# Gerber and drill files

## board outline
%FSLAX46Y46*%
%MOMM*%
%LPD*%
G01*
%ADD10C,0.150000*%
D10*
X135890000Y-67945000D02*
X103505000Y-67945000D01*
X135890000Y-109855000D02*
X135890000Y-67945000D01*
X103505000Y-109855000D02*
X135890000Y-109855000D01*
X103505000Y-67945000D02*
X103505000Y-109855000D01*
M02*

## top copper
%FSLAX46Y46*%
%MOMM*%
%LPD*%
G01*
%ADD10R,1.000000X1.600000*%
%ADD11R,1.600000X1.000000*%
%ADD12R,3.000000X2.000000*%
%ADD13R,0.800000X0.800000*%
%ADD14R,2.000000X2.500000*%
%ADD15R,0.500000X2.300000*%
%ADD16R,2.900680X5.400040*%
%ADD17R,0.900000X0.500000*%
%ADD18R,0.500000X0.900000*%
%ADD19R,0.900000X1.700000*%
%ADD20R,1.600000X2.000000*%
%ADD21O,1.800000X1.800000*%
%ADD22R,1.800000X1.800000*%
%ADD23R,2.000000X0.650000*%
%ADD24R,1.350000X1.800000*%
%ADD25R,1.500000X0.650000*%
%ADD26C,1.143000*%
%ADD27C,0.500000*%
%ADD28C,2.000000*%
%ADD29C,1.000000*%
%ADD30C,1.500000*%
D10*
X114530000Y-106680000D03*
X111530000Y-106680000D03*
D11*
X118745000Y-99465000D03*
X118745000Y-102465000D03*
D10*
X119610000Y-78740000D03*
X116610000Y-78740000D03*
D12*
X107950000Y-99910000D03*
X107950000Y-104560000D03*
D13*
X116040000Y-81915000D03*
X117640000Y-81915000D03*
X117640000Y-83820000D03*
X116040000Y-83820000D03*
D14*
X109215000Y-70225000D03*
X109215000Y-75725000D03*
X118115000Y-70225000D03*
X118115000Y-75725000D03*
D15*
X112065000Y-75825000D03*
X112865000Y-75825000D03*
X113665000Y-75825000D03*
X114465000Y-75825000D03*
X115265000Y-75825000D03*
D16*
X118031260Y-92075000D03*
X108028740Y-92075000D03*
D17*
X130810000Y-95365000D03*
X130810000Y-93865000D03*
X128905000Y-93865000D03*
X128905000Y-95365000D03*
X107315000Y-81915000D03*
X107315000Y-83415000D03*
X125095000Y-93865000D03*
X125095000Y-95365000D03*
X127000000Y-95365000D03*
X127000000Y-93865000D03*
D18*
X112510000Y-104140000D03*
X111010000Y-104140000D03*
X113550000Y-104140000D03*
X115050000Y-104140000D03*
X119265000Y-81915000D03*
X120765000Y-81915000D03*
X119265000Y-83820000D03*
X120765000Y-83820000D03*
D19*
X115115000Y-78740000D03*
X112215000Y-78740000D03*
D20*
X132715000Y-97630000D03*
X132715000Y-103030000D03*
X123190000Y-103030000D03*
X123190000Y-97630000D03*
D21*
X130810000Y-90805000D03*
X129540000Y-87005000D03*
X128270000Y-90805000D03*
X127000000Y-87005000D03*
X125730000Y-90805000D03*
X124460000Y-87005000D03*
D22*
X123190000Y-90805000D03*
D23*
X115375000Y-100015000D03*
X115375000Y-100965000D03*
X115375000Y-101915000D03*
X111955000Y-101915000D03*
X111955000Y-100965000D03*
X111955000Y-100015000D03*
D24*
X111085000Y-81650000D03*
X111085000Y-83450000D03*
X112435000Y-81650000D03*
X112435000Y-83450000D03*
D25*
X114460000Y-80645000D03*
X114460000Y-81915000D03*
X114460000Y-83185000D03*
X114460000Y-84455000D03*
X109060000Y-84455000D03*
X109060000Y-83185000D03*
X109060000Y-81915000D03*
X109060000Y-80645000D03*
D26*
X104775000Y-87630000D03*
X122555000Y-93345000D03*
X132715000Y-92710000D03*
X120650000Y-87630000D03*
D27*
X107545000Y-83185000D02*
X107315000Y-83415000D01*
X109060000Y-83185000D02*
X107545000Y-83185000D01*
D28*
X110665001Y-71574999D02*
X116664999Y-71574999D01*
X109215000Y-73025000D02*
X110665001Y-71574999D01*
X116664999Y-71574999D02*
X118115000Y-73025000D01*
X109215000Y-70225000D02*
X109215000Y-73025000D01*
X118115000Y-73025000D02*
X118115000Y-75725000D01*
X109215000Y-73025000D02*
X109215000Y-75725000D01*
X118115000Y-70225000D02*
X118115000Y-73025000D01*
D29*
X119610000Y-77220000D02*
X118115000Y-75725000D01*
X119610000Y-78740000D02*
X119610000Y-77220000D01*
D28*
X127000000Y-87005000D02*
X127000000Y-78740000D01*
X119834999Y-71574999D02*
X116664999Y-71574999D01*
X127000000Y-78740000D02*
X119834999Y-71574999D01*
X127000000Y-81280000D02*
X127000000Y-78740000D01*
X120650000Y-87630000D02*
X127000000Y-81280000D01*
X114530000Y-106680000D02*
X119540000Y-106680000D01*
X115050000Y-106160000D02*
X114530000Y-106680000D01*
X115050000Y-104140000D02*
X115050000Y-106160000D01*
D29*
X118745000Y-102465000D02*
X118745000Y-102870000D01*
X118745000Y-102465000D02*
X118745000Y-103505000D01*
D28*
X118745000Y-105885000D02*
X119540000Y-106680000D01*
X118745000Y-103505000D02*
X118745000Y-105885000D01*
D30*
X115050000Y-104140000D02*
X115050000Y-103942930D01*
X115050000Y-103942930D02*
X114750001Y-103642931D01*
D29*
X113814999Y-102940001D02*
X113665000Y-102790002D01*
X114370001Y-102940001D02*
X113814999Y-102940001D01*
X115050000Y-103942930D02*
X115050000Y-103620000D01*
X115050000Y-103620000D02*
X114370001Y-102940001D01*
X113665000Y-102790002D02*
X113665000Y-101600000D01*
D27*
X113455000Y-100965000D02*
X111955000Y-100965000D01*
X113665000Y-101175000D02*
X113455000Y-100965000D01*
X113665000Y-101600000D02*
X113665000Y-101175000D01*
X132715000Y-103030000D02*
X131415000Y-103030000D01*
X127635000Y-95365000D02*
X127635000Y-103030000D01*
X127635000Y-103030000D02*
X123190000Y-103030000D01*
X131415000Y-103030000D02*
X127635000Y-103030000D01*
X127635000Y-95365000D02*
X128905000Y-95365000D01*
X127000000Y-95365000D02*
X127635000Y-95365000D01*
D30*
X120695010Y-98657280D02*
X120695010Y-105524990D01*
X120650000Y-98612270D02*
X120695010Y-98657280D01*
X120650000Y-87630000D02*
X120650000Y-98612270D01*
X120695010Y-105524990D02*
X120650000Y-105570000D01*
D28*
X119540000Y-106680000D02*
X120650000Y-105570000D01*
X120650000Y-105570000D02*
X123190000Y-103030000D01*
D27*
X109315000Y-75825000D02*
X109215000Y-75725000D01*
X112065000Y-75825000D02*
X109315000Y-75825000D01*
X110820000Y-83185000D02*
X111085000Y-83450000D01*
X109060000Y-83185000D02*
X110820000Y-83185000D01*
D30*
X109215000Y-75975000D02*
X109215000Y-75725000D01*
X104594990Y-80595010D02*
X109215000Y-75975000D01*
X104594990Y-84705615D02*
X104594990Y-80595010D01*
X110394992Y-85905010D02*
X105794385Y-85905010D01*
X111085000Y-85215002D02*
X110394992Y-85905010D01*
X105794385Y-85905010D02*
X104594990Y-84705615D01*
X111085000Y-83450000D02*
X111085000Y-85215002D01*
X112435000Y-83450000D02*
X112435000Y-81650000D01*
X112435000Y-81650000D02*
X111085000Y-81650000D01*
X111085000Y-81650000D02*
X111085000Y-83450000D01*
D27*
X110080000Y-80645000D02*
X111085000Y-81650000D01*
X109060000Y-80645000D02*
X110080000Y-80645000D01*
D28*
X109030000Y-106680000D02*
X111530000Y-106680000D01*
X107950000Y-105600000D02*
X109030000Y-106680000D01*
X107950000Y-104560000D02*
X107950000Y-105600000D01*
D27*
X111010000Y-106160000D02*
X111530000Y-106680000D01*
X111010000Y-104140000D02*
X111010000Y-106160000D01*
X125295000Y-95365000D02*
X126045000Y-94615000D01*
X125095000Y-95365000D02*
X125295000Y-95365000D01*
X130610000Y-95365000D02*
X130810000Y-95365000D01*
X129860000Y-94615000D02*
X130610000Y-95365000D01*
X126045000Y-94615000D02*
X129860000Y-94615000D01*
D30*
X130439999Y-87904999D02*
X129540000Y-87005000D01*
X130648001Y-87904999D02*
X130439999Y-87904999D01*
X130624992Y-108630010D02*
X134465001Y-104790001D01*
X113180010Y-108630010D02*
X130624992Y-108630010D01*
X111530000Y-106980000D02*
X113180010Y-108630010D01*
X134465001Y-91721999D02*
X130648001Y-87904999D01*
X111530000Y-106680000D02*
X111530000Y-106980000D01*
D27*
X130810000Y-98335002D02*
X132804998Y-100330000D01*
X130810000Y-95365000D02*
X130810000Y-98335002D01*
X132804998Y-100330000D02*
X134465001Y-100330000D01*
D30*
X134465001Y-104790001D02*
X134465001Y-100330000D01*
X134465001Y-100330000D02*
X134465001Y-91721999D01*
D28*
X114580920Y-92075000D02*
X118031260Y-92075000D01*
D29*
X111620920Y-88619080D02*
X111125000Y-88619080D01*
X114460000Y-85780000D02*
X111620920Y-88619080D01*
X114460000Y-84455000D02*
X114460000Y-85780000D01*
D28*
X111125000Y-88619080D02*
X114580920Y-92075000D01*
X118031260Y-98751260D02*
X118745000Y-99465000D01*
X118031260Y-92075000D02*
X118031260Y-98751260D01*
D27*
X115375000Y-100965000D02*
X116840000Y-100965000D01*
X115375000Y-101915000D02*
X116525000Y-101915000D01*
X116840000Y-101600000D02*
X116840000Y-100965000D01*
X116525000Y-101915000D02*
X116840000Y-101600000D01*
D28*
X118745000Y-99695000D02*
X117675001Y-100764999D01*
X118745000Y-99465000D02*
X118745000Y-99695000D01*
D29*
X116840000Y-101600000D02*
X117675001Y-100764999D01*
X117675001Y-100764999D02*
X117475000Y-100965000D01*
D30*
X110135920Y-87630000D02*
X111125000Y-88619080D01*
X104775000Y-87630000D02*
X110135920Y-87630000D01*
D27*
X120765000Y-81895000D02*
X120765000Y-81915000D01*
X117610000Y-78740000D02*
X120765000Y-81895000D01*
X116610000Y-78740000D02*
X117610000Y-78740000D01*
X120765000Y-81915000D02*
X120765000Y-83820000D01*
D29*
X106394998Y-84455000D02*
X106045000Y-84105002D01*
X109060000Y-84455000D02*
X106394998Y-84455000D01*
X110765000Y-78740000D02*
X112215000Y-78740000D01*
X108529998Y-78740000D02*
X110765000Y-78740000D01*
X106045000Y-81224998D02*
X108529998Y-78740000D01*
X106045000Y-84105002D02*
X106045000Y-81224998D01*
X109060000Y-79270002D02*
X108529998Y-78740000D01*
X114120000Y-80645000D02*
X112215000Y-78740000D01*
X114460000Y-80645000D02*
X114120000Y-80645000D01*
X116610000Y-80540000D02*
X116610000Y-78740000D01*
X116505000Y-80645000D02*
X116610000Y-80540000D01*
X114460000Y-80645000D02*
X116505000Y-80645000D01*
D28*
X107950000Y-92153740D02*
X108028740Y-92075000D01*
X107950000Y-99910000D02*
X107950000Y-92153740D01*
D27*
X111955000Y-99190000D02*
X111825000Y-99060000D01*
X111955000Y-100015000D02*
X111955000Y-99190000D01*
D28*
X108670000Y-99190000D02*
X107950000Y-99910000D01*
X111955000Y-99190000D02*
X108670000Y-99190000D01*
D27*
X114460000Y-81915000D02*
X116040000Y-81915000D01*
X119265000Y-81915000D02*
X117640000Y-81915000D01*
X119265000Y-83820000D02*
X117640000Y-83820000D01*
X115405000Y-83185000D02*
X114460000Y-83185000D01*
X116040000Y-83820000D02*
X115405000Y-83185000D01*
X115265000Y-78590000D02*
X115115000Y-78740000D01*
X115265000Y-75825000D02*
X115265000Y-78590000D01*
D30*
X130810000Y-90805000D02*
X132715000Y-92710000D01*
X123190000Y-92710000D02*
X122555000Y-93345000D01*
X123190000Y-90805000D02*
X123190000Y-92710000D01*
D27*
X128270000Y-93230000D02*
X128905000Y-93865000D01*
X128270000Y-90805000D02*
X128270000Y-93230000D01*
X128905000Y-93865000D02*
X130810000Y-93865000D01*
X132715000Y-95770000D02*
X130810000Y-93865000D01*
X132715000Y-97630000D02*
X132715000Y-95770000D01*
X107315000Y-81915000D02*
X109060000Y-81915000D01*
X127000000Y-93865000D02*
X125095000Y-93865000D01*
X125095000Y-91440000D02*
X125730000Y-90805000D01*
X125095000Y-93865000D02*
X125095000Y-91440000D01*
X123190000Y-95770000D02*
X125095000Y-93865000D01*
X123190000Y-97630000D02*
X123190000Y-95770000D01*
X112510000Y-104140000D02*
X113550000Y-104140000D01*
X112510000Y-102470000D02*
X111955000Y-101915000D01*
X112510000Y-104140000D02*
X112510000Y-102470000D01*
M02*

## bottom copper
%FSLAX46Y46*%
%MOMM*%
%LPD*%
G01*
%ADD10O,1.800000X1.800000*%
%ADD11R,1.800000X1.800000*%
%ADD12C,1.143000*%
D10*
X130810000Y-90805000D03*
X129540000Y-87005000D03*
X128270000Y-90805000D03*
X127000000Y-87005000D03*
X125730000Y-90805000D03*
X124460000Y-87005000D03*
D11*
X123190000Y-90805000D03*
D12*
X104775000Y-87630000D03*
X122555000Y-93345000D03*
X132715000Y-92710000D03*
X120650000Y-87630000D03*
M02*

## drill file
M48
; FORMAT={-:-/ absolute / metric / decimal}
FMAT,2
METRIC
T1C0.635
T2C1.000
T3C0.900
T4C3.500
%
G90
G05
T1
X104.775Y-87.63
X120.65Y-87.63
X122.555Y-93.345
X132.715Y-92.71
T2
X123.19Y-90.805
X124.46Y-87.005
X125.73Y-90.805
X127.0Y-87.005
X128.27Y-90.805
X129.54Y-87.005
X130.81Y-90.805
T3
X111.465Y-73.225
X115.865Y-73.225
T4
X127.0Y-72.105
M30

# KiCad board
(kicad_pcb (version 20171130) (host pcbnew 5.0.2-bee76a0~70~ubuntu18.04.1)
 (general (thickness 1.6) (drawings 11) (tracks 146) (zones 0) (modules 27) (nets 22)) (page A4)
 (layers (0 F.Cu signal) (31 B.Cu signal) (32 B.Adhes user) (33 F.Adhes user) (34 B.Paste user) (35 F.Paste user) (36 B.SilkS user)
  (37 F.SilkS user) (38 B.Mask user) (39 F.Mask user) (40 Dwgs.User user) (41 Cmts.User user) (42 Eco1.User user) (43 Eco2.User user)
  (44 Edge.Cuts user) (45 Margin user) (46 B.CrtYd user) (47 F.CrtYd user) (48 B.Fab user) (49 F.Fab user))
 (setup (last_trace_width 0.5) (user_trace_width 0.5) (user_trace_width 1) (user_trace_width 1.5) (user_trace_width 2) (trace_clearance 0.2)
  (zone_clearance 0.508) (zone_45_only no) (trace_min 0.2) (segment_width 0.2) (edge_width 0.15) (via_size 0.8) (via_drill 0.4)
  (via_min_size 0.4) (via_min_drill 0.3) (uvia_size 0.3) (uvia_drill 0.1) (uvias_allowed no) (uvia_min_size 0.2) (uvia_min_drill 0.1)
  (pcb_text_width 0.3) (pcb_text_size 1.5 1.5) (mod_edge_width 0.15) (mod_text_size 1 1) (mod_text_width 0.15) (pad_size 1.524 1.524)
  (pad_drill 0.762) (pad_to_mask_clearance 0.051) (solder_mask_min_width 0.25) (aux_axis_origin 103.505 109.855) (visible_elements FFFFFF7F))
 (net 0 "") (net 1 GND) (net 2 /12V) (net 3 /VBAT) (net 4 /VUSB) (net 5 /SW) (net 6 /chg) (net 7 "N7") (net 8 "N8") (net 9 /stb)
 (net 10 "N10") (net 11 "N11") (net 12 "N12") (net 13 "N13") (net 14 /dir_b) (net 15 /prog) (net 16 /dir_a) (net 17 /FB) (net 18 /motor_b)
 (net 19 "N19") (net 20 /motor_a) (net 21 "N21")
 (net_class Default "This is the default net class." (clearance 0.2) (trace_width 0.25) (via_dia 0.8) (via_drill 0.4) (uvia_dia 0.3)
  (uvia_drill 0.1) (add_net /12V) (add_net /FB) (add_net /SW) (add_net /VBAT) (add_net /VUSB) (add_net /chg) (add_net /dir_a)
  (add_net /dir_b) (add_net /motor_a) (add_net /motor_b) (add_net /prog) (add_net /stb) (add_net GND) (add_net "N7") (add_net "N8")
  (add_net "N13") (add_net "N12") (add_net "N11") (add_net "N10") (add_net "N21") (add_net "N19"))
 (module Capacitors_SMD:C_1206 (layer F.Cu) (at 113.03 106.68)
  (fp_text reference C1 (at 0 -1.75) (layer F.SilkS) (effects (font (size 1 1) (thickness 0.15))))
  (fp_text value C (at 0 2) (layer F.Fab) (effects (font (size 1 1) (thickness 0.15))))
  (pad 2 smd rect (at 1.5 0) (size 1 1.6) (layers F.Cu F.Paste F.Mask) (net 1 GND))
  (pad 1 smd rect (at -1.5 0) (size 1 1.6) (layers F.Cu F.Paste F.Mask) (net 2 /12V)))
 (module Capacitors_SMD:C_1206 (layer F.Cu) (at 118.745 100.965 270)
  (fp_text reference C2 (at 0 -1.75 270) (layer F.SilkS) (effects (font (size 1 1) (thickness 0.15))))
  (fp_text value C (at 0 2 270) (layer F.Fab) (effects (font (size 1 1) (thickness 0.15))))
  (pad 1 smd rect (at -1.5 0 270) (size 1 1.6) (layers F.Cu F.Paste F.Mask) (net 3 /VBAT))
  (pad 2 smd rect (at 1.5 0 270) (size 1 1.6) (layers F.Cu F.Paste F.Mask) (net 1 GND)))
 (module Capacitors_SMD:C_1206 (layer F.Cu) (at 118.11 78.74)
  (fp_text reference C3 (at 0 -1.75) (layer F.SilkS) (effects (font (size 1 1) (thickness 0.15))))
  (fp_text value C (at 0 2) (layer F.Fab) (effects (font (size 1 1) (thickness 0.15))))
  (pad 2 smd rect (at 1.5 0) (size 1 1.6) (layers F.Cu F.Paste F.Mask) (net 1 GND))
  (pad 1 smd rect (at -1.5 0) (size 1 1.6) (layers F.Cu F.Paste F.Mask) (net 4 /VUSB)))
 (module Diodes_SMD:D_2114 (layer F.Cu) (at 107.95 102.235 90)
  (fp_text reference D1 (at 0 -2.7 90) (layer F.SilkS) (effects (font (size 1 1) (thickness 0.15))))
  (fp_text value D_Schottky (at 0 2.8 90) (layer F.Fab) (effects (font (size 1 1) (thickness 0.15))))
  (pad 2 smd rect (at 2.325 0 90) (size 2 3) (layers F.Cu F.Paste F.Mask) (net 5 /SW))
  (pad 1 smd rect (at -2.325 0 90) (size 2 3) (layers F.Cu F.Paste F.Mask) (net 2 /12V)))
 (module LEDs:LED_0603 (layer F.Cu) (at 116.84 81.915)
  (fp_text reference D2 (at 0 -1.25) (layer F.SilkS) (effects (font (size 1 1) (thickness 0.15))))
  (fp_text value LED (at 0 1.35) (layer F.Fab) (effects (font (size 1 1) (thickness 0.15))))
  (pad 1 smd rect (at -0.8 0 180) (size 0.8 0.8) (layers F.Cu F.Paste F.Mask) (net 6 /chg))
  (pad 2 smd rect (at 0.8 0 180) (size 0.8 0.8) (layers F.Cu F.Paste F.Mask) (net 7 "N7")))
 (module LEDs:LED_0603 (layer F.Cu) (at 116.84 83.82)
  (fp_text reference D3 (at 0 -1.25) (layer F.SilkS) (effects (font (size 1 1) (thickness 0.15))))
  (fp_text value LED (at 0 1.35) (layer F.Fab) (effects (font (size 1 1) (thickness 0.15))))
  (pad 2 smd rect (at 0.8 0 180) (size 0.8 0.8) (layers F.Cu F.Paste F.Mask) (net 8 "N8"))
  (pad 1 smd rect (at -0.8 0 180) (size 0.8 0.8) (layers F.Cu F.Paste F.Mask) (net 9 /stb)))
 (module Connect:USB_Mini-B (layer F.Cu) (at 113.665 73.025 270)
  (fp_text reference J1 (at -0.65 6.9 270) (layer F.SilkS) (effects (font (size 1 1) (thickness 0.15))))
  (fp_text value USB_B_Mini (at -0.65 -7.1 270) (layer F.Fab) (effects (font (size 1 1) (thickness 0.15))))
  (pad "" np_thru_hole circle (at 0.2 2.2 270) (size 0.9 0.9) (drill 0.9) (layers *.Cu *.Mask))
  (pad "" np_thru_hole circle (at 0.2 -2.2 270) (size 0.9 0.9) (drill 0.9) (layers *.Cu *.Mask))
  (pad 6 smd rect (at -2.8 4.45 270) (size 2.5 2) (layers F.Cu F.Paste F.Mask) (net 1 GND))
  (pad 6 smd rect (at 2.7 4.45 270) (size 2.5 2) (layers F.Cu F.Paste F.Mask) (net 1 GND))
  (pad 6 smd rect (at -2.8 -4.45 270) (size 2.5 2) (layers F.Cu F.Paste F.Mask) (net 1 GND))
  (pad 6 smd rect (at 2.7 -4.45 270) (size 2.5 2) (layers F.Cu F.Paste F.Mask) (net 1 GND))
  (pad 5 smd rect (at 2.8 1.6 270) (size 2.3 0.5) (layers F.Cu F.Paste F.Mask) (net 1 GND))
  (pad 4 smd rect (at 2.8 0.8 270) (size 2.3 0.5) (layers F.Cu F.Paste F.Mask) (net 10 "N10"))
  (pad 3 smd rect (at 2.8 0 270) (size 2.3 0.5) (layers F.Cu F.Paste F.Mask) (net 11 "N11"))
  (pad 2 smd rect (at 2.8 -0.8 270) (size 2.3 0.5) (layers F.Cu F.Paste F.Mask) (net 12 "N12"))
  (pad 1 smd rect (at 2.8 -1.6 270) (size 2.3 0.5) (layers F.Cu F.Paste F.Mask) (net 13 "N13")))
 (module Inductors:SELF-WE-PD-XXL (layer F.Cu) (at 113.03 92.075)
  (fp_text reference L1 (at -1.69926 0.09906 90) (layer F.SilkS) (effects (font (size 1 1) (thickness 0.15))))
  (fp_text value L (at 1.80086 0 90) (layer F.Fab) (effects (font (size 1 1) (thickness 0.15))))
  (pad 2 smd rect (at 5.00126 0) (size 2.90068 5.40004) (layers F.Cu F.Paste F.Mask) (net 3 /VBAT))
  (pad 1 smd rect (at -5.00126 0) (size 2.90068 5.40004) (layers F.Cu F.Paste F.Mask) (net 5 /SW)))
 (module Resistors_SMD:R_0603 (layer F.Cu) (at 130.81 94.615 90)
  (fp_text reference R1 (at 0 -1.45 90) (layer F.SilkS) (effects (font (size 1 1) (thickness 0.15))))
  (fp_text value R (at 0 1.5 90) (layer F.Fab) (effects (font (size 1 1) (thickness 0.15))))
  (pad 1 smd rect (at -0.75 0 90) (size 0.5 0.9) (layers F.Cu F.Paste F.Mask) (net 2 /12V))
  (pad 2 smd rect (at 0.75 0 90) (size 0.5 0.9) (layers F.Cu F.Paste F.Mask) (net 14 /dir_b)))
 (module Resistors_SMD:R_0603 (layer F.Cu) (at 128.905 94.615 270)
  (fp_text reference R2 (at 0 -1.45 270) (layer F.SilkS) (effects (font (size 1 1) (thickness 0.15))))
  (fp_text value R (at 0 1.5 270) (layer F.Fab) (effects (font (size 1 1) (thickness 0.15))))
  (pad 1 smd rect (at -0.75 0 270) (size 0.5 0.9) (layers F.Cu F.Paste F.Mask) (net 14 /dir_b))
  (pad 2 smd rect (at 0.75 0 270) (size 0.5 0.9) (layers F.Cu F.Paste F.Mask) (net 1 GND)))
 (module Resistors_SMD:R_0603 (layer F.Cu) (at 107.315 82.665 270)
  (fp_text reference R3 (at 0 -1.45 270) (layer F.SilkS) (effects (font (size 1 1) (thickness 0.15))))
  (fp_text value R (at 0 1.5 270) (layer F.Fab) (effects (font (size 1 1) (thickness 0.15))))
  (pad 1 smd rect (at -0.75 0 270) (size 0.5 0.9) (layers F.Cu F.Paste F.Mask) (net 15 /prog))
  (pad 2 smd rect (at 0.75 0 270) (size 0.5 0.9) (layers F.Cu F.Paste F.Mask) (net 1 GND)))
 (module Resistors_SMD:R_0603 (layer F.Cu) (at 125.095 94.615 90)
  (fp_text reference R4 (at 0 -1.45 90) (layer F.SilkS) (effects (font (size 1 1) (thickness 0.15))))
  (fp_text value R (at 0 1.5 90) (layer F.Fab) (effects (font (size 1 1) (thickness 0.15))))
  (pad 2 smd rect (at 0.75 0 90) (size 0.5 0.9) (layers F.Cu F.Paste F.Mask) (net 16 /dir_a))
  (pad 1 smd rect (at -0.75 0 90) (size 0.5 0.9) (layers F.Cu F.Paste F.Mask) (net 2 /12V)))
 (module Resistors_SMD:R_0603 (layer F.Cu) (at 127 94.615 270)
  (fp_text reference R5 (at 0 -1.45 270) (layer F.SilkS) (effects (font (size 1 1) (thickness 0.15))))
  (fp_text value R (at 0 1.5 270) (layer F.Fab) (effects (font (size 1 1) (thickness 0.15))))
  (pad 2 smd rect (at 0.75 0 270) (size 0.5 0.9) (layers F.Cu F.Paste F.Mask) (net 1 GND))
  (pad 1 smd rect (at -0.75 0 270) (size 0.5 0.9) (layers F.Cu F.Paste F.Mask) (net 16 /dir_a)))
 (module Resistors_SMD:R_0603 (layer F.Cu) (at 111.76 104.14)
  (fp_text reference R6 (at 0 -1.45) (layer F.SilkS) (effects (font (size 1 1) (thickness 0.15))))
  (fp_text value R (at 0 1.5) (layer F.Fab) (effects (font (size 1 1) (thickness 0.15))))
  (pad 2 smd rect (at 0.75 0) (size 0.5 0.9) (layers F.Cu F.Paste F.Mask) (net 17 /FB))
  (pad 1 smd rect (at -0.75 0) (size 0.5 0.9) (layers F.Cu F.Paste F.Mask) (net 2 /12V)))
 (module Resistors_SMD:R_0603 (layer F.Cu) (at 114.3 104.14)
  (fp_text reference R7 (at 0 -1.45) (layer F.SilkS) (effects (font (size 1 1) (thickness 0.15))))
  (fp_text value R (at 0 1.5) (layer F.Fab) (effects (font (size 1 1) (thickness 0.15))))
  (pad 1 smd rect (at -0.75 0) (size 0.5 0.9) (layers F.Cu F.Paste F.Mask) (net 17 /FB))
  (pad 2 smd rect (at 0.75 0) (size 0.5 0.9) (layers F.Cu F.Paste F.Mask) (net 1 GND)))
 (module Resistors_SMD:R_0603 (layer F.Cu) (at 120.015 81.915 180)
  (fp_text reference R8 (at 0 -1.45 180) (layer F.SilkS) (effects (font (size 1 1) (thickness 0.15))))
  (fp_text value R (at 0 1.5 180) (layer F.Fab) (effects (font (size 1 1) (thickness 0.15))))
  (pad 2 smd rect (at 0.75 0 180) (size 0.5 0.9) (layers F.Cu F.Paste F.Mask) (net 7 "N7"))
  (pad 1 smd rect (at -0.75 0 180) (size 0.5 0.9) (layers F.Cu F.Paste F.Mask) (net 4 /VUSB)))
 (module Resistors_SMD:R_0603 (layer F.Cu) (at 120.015 83.82 180)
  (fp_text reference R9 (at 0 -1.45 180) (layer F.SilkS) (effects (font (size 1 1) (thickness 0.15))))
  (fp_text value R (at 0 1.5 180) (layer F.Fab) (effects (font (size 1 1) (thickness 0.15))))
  (pad 2 smd rect (at 0.75 0 180) (size 0.5 0.9) (layers F.Cu F.Paste F.Mask) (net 8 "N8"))
  (pad 1 smd rect (at -0.75 0 180) (size 0.5 0.9) (layers F.Cu F.Paste F.Mask) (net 4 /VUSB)))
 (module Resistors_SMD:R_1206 (layer F.Cu) (at 113.665 78.74)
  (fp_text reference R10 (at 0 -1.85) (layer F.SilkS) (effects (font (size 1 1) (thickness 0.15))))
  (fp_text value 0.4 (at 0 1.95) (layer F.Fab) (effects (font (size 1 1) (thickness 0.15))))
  (pad 2 smd rect (at 1.45 0) (size 0.9 1.7) (layers F.Cu F.Paste F.Mask) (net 13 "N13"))
  (pad 1 smd rect (at -1.45 0) (size 0.9 1.7) (layers F.Cu F.Paste F.Mask) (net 4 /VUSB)))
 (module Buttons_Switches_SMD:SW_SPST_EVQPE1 (layer F.Cu) (at 132.715 100.33 270)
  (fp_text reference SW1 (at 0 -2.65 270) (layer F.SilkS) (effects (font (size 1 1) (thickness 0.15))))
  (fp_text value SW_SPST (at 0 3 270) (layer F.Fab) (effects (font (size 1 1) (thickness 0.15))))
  (pad 1 smd rect (at -2.7 0 270) (size 2 1.6) (layers F.Cu F.Paste F.Mask) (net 14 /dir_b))
  (pad 2 smd rect (at 2.7 0 270) (size 2 1.6) (layers F.Cu F.Paste F.Mask) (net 1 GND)))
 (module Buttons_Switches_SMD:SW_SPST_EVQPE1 (layer F.Cu) (at 123.19 100.33 270)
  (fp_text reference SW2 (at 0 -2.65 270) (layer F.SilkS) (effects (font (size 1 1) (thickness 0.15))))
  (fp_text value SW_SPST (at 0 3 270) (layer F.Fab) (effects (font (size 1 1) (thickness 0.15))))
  (pad 2 smd rect (at 2.7 0 270) (size 2 1.6) (layers F.Cu F.Paste F.Mask) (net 1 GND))
  (pad 1 smd rect (at -2.7 0 270) (size 2 1.6) (layers F.Cu F.Paste F.Mask) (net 16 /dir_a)))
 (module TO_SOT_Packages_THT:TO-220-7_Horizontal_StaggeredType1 (layer F.Cu) (at 123.19 90.805)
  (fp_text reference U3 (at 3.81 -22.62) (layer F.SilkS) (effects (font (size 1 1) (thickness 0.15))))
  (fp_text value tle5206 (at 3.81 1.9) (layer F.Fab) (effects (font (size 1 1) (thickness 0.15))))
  (pad 7 thru_hole oval (at 7.62 0) (size 1.8 1.8) (drill 1) (layers *.Cu *.Mask) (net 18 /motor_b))
  (pad 6 thru_hole oval (at 6.35 -3.8) (size 1.8 1.8) (drill 1) (layers *.Cu *.Mask) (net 2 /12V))
  (pad 5 thru_hole oval (at 5.08 0) (size 1.8 1.8) (drill 1) (layers *.Cu *.Mask) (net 14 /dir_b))
  (pad 4 thru_hole oval (at 3.81 -3.8) (size 1.8 1.8) (drill 1) (layers *.Cu *.Mask) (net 1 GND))
  (pad 3 thru_hole oval (at 2.54 0) (size 1.8 1.8) (drill 1) (layers *.Cu *.Mask) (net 16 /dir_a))
  (pad 2 thru_hole oval (at 1.27 -3.8) (size 1.8 1.8) (drill 1) (layers *.Cu *.Mask) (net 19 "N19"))
  (pad 1 thru_hole rect (at 0 0) (size 1.8 1.8) (drill 1) (layers *.Cu *.Mask) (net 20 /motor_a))
  (pad 0 np_thru_hole oval (at 3.81 -18.7) (size 3.5 3.5) (drill 3.5) (layers *.Cu *.Mask)))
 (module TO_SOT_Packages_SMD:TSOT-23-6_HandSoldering (layer F.Cu) (at 113.665 100.965)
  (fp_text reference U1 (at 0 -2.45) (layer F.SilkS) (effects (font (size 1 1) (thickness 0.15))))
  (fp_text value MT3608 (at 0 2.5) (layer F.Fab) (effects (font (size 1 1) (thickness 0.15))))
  (pad 6 smd rect (at 1.71 -0.95) (size 2 0.65) (layers F.Cu F.Paste F.Mask) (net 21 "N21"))
  (pad 5 smd rect (at 1.71 0) (size 2 0.65) (layers F.Cu F.Paste F.Mask) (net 3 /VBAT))
  (pad 4 smd rect (at 1.71 0.95) (size 2 0.65) (layers F.Cu F.Paste F.Mask) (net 3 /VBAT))
  (pad 3 smd rect (at -1.71 0.95) (size 2 0.65) (layers F.Cu F.Paste F.Mask) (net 17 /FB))
  (pad 2 smd rect (at -1.71 0) (size 2 0.65) (layers F.Cu F.Paste F.Mask) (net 1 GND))
  (pad 1 smd rect (at -1.71 -0.95) (size 2 0.65) (layers F.Cu F.Paste F.Mask) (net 5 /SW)))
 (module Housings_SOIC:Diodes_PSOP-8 (layer F.Cu) (at 111.76 82.55)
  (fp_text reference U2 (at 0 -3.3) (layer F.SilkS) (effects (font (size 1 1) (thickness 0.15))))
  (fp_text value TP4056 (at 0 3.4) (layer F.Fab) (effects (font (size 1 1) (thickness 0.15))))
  (pad 9 smd rect (at -0.675 -0.9) (size 1.35 1.8) (layers F.Cu F.Paste F.Mask) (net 1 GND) (solder_paste_margin_ratio -0.2))
  (pad 9 smd rect (at -0.675 0.9) (size 1.35 1.8) (layers F.Cu F.Paste F.Mask) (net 1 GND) (solder_paste_margin_ratio -0.2))
  (pad 9 smd rect (at 0.675 -0.9) (size 1.35 1.8) (layers F.Cu F.Paste F.Mask) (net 1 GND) (solder_paste_margin_ratio -0.2))
  (pad 9 smd rect (at 0.675 0.9) (size 1.35 1.8) (layers F.Cu F.Paste F.Mask) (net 1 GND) (solder_paste_margin_ratio -0.2))
  (pad 8 smd rect (at 2.7 -1.905) (size 1.5 0.65) (layers F.Cu F.Paste F.Mask) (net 4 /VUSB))
  (pad 7 smd rect (at 2.7 -0.635) (size 1.5 0.65) (layers F.Cu F.Paste F.Mask) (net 6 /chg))
  (pad 6 smd rect (at 2.7 0.635) (size 1.5 0.65) (layers F.Cu F.Paste F.Mask) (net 9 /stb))
  (pad 5 smd rect (at 2.7 1.905) (size 1.5 0.65) (layers F.Cu F.Paste F.Mask) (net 3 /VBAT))
  (pad 4 smd rect (at -2.7 1.905) (size 1.5 0.65) (layers F.Cu F.Paste F.Mask) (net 4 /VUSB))
  (pad 3 smd rect (at -2.7 0.635) (size 1.5 0.65) (layers F.Cu F.Paste F.Mask) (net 1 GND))
  (pad 2 smd rect (at -2.7 -0.635) (size 1.5 0.65) (layers F.Cu F.Paste F.Mask) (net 15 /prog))
  (pad 1 smd rect (at -2.7 -1.905) (size 1.5 0.65) (layers F.Cu F.Paste F.Mask) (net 1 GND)))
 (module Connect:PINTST (layer F.Cu) (at 104.775 87.63)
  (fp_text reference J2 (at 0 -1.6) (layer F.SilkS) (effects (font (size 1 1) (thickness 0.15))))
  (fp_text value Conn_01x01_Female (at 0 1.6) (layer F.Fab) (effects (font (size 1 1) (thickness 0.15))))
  (pad 1 thru_hole circle (at 0 0) (size 1.143 1.143) (drill 0.635) (layers *.Cu *.Mask) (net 3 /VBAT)))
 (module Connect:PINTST (layer F.Cu) (at 122.555 93.345)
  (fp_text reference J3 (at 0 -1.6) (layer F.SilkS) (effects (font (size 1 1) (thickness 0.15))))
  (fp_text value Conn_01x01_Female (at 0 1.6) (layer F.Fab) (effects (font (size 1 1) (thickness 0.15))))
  (pad 1 thru_hole circle (at 0 0) (size 1.143 1.143) (drill 0.635) (layers *.Cu *.Mask) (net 20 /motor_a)))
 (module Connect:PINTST (layer F.Cu) (at 132.715 92.71)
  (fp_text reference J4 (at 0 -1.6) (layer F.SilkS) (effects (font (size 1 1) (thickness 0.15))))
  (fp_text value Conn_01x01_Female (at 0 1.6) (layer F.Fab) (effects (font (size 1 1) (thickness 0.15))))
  (pad 1 thru_hole circle (at 0 0) (size 1.143 1.143) (drill 0.635) (layers *.Cu *.Mask) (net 18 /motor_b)))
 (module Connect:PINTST (layer F.Cu) (at 120.65 87.63)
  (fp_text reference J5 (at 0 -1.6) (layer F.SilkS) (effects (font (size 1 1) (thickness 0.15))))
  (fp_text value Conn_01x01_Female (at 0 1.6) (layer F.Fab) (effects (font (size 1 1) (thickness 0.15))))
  (pad 1 thru_hole circle (at 0 0) (size 1.143 1.143) (drill 0.635) (layers *.Cu *.Mask) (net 1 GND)))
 (gr_line (start 135.89 67.945) (end 103.505 67.945) (layer Edge.Cuts) (width 0.15))
 (gr_line (start 135.89 109.855) (end 135.89 67.945) (layer Edge.Cuts) (width 0.15))
 (gr_line (start 103.505 109.855) (end 135.89 109.855) (layer Edge.Cuts) (width 0.15))
 (gr_line (start 103.505 67.945) (end 103.505 109.855) (layer Edge.Cuts) (width 0.15))
 (segment (start 107.545 83.185) (end 107.315 83.415) (width 0.5) (layer F.Cu) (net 1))
 (segment (start 109.06 83.185) (end 107.545 83.185) (width 0.5) (layer F.Cu) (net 1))
 (segment (start 110.665001 71.574999) (end 116.664999 71.574999) (width 2) (layer F.Cu) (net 1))
 (segment (start 109.215 73.025) (end 110.665001 71.574999) (width 2) (layer F.Cu) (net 1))
 (segment (start 116.664999 71.574999) (end 118.115 73.025) (width 2) (layer F.Cu) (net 1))
 (segment (start 109.215 70.225) (end 109.215 73.025) (width 2) (layer F.Cu) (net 1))
 (segment (start 118.115 73.025) (end 118.115 75.725) (width 2) (layer F.Cu) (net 1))
 (segment (start 109.215 73.025) (end 109.215 75.725) (width 2) (layer F.Cu) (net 1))
 (segment (start 118.115 70.225) (end 118.115 73.025) (width 2) (layer F.Cu) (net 1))
 (segment (start 119.61 77.22) (end 118.115 75.725) (width 1) (layer F.Cu) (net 1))
 (segment (start 119.61 78.74) (end 119.61 77.22) (width 1) (layer F.Cu) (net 1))
 (segment (start 127 87.005) (end 127 78.74) (width 2) (layer F.Cu) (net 1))
 (segment (start 119.834999 71.574999) (end 116.664999 71.574999) (width 2) (layer F.Cu) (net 1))
 (segment (start 127 78.74) (end 119.834999 71.574999) (width 2) (layer F.Cu) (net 1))
 (segment (start 127 81.28) (end 127 78.74) (width 2) (layer F.Cu) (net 1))
 (segment (start 120.65 87.63) (end 127 81.28) (width 2) (layer F.Cu) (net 1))
 (segment (start 114.53 106.68) (end 119.54 106.68) (width 2) (layer F.Cu) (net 1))
 (segment (start 115.05 106.16) (end 114.53 106.68) (width 2) (layer F.Cu) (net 1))
 (segment (start 115.05 104.14) (end 115.05 106.16) (width 2) (layer F.Cu) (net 1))
 (segment (start 118.745 102.465) (end 118.745 102.87) (width 1) (layer F.Cu) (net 1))
 (segment (start 118.745 102.465) (end 118.745 103.505) (width 1) (layer F.Cu) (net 1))
 (segment (start 118.745 105.885) (end 119.54 106.68) (width 2) (layer F.Cu) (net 1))
 (segment (start 118.745 103.505) (end 118.745 105.885) (width 2) (layer F.Cu) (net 1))
 (segment (start 115.05 104.14) (end 115.05 103.94293) (width 1.5) (layer F.Cu) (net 1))
 (segment (start 115.05 103.94293) (end 114.750001 103.642931) (width 1.5) (layer F.Cu) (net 1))
 (segment (start 113.814999 102.940001) (end 113.665 102.790002) (width 1) (layer F.Cu) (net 1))
 (segment (start 114.370001 102.940001) (end 113.814999 102.940001) (width 1) (layer F.Cu) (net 1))
 (segment (start 115.05 103.94293) (end 115.05 103.62) (width 1) (layer F.Cu) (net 1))
 (segment (start 115.05 103.62) (end 114.370001 102.940001) (width 1) (layer F.Cu) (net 1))
 (segment (start 113.665 102.790002) (end 113.665 101.6) (width 1) (layer F.Cu) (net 1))
 (segment (start 113.455 100.965) (end 111.955 100.965) (width 0.5) (layer F.Cu) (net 1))
 (segment (start 113.665 101.175) (end 113.455 100.965) (width 0.5) (layer F.Cu) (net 1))
 (segment (start 113.665 101.6) (end 113.665 101.175) (width 0.5) (layer F.Cu) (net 1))
 (segment (start 132.715 103.03) (end 131.415 103.03) (width 0.5) (layer F.Cu) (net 1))
 (segment (start 127.635 95.365) (end 127.635 103.03) (width 0.5) (layer F.Cu) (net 1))
 (segment (start 127.635 103.03) (end 123.19 103.03) (width 0.5) (layer F.Cu) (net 1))
 (segment (start 131.415 103.03) (end 127.635 103.03) (width 0.5) (layer F.Cu) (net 1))
 (segment (start 127.635 95.365) (end 128.905 95.365) (width 0.5) (layer F.Cu) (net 1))
 (segment (start 127 95.365) (end 127.635 95.365) (width 0.5) (layer F.Cu) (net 1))
 (segment (start 120.69501 98.65728) (end 120.69501 105.52499) (width 1.5) (layer F.Cu) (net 1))
 (segment (start 120.65 98.61227) (end 120.69501 98.65728) (width 1.5) (layer F.Cu) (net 1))
 (segment (start 120.65 87.63) (end 120.65 98.61227) (width 1.5) (layer F.Cu) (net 1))
 (segment (start 120.69501 105.52499) (end 120.65 105.57) (width 1.5) (layer F.Cu) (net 1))
 (segment (start 119.54 106.68) (end 120.65 105.57) (width 2) (layer F.Cu) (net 1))
 (segment (start 120.65 105.57) (end 123.19 103.03) (width 2) (layer F.Cu) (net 1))
 (segment (start 109.315 75.825) (end 109.215 75.725) (width 0.5) (layer F.Cu) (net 1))
 (segment (start 112.065 75.825) (end 109.315 75.825) (width 0.5) (layer F.Cu) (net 1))
 (segment (start 110.82 83.185) (end 111.085 83.45) (width 0.5) (layer F.Cu) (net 1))
 (segment (start 109.06 83.185) (end 110.82 83.185) (width 0.5) (layer F.Cu) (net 1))
 (segment (start 109.215 75.975) (end 109.215 75.725) (width 1.5) (layer F.Cu) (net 1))
 (segment (start 104.59499 80.59501) (end 109.215 75.975) (width 1.5) (layer F.Cu) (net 1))
 (segment (start 104.59499 84.705615) (end 104.59499 80.59501) (width 1.5) (layer F.Cu) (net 1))
 (segment (start 110.394992 85.90501) (end 105.794385 85.90501) (width 1.5) (layer F.Cu) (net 1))
 (segment (start 111.085 85.215002) (end 110.394992 85.90501) (width 1.5) (layer F.Cu) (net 1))
 (segment (start 105.794385 85.90501) (end 104.59499 84.705615) (width 1.5) (layer F.Cu) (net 1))
 (segment (start 111.085 83.45) (end 111.085 85.215002) (width 1.5) (layer F.Cu) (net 1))
 (segment (start 112.435 83.45) (end 112.435 81.65) (width 1.5) (layer F.Cu) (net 1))
 (segment (start 112.435 81.65) (end 111.085 81.65) (width 1.5) (layer F.Cu) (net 1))
 (segment (start 111.085 81.65) (end 111.085 83.45) (width 1.5) (layer F.Cu) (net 1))
 (segment (start 110.08 80.645) (end 111.085 81.65) (width 0.5) (layer F.Cu) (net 1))
 (segment (start 109.06 80.645) (end 110.08 80.645) (width 0.5) (layer F.Cu) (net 1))
 (segment (start 109.03 106.68) (end 111.53 106.68) (width 2) (layer F.Cu) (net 2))
 (segment (start 107.95 105.6) (end 109.03 106.68) (width 2) (layer F.Cu) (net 2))
 (segment (start 107.95 104.56) (end 107.95 105.6) (width 2) (layer F.Cu) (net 2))
 (segment (start 111.01 106.16) (end 111.53 106.68) (width 0.5) (layer F.Cu) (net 2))
 (segment (start 111.01 104.14) (end 111.01 106.16) (width 0.5) (layer F.Cu) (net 2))
 (segment (start 125.295 95.365) (end 126.045 94.615) (width 0.5) (layer F.Cu) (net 2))
 (segment (start 125.095 95.365) (end 125.295 95.365) (width 0.5) (layer F.Cu) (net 2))
 (segment (start 130.61 95.365) (end 130.81 95.365) (width 0.5) (layer F.Cu) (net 2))
 (segment (start 129.86 94.615) (end 130.61 95.365) (width 0.5) (layer F.Cu) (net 2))
 (segment (start 126.045 94.615) (end 129.86 94.615) (width 0.5) (layer F.Cu) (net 2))
 (segment (start 130.439999 87.904999) (end 129.54 87.005) (width 1.5) (layer F.Cu) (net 2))
 (segment (start 130.648001 87.904999) (end 130.439999 87.904999) (width 1.5) (layer F.Cu) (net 2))
 (segment (start 130.624992 108.63001) (end 134.465001 104.790001) (width 1.5) (layer F.Cu) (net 2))
 (segment (start 113.18001 108.63001) (end 130.624992 108.63001) (width 1.5) (layer F.Cu) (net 2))
 (segment (start 111.53 106.98) (end 113.18001 108.63001) (width 1.5) (layer F.Cu) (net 2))
 (segment (start 134.465001 91.721999) (end 130.648001 87.904999) (width 1.5) (layer F.Cu) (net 2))
 (segment (start 111.53 106.68) (end 111.53 106.98) (width 1.5) (layer F.Cu) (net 2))
 (segment (start 130.81 98.335002) (end 132.804998 100.33) (width 0.5) (layer F.Cu) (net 2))
 (segment (start 130.81 95.365) (end 130.81 98.335002) (width 0.5) (layer F.Cu) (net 2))
 (segment (start 132.804998 100.33) (end 134.465001 100.33) (width 0.5) (layer F.Cu) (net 2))
 (segment (start 134.465001 104.790001) (end 134.465001 100.33) (width 1.5) (layer F.Cu) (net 2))
 (segment (start 134.465001 100.33) (end 134.465001 91.721999) (width 1.5) (layer F.Cu) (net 2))
 (segment (start 114.58092 92.075) (end 118.03126 92.075) (width 2) (layer F.Cu) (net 3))
 (segment (start 111.62092 88.61908) (end 111.125 88.61908) (width 1) (layer F.Cu) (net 3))
 (segment (start 114.46 85.78) (end 111.62092 88.61908) (width 1) (layer F.Cu) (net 3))
 (segment (start 114.46 84.455) (end 114.46 85.78) (width 1) (layer F.Cu) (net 3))
 (segment (start 111.125 88.61908) (end 114.58092 92.075) (width 2) (layer F.Cu) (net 3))
 (segment (start 118.03126 98.75126) (end 118.745 99.465) (width 2) (layer F.Cu) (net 3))
 (segment (start 118.03126 92.075) (end 118.03126 98.75126) (width 2) (layer F.Cu) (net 3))
 (segment (start 115.375 100.965) (end 116.84 100.965) (width 0.5) (layer F.Cu) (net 3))
 (segment (start 115.375 101.915) (end 116.525 101.915) (width 0.5) (layer F.Cu) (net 3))
 (segment (start 116.84 101.6) (end 116.84 100.965) (width 0.5) (layer F.Cu) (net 3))
 (segment (start 116.525 101.915) (end 116.84 101.6) (width 0.5) (layer F.Cu) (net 3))
 (segment (start 118.745 99.695) (end 117.675001 100.764999) (width 2) (layer F.Cu) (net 3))
 (segment (start 118.745 99.465) (end 118.745 99.695) (width 2) (layer F.Cu) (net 3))
 (segment (start 116.84 101.6) (end 117.675001 100.764999) (width 1) (layer F.Cu) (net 3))
 (segment (start 117.675001 100.764999) (end 117.475 100.965) (width 1) (layer F.Cu) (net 3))
 (segment (start 110.13592 87.63) (end 111.125 88.61908) (width 1.5) (layer F.Cu) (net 3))
 (segment (start 104.775 87.63) (end 110.13592 87.63) (width 1.5) (layer F.Cu) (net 3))
 (segment (start 120.765 81.895) (end 120.765 81.915) (width 0.5) (layer F.Cu) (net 4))
 (segment (start 117.61 78.74) (end 120.765 81.895) (width 0.5) (layer F.Cu) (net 4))
 (segment (start 116.61 78.74) (end 117.61 78.74) (width 0.5) (layer F.Cu) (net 4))
 (segment (start 120.765 81.915) (end 120.765 83.82) (width 0.5) (layer F.Cu) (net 4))
 (segment (start 106.394998 84.455) (end 106.045 84.105002) (width 1) (layer F.Cu) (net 4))
 (segment (start 109.06 84.455) (end 106.394998 84.455) (width 1) (layer F.Cu) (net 4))
 (segment (start 110.765 78.74) (end 112.215 78.74) (width 1) (layer F.Cu) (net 4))
 (segment (start 108.529998 78.74) (end 110.765 78.74) (width 1) (layer F.Cu) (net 4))
 (segment (start 106.045 81.224998) (end 108.529998 78.74) (width 1) (layer F.Cu) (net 4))
 (segment (start 106.045 84.105002) (end 106.045 81.224998) (width 1) (layer F.Cu) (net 4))
 (segment (start 109.06 79.270002) (end 108.529998 78.74) (width 1) (layer F.Cu) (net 4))
 (segment (start 114.12 80.645) (end 112.215 78.74) (width 1) (layer F.Cu) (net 4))
 (segment (start 114.46 80.645) (end 114.12 80.645) (width 1) (layer F.Cu) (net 4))
 (segment (start 116.61 80.54) (end 116.61 78.74) (width 1) (layer F.Cu) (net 4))
 (segment (start 116.505 80.645) (end 116.61 80.54) (width 1) (layer F.Cu) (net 4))
 (segment (start 114.46 80.645) (end 116.505 80.645) (width 1) (layer F.Cu) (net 4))
 (segment (start 107.95 92.15374) (end 108.02874 92.075) (width 2) (layer F.Cu) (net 5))
 (segment (start 107.95 99.91) (end 107.95 92.15374) (width 2) (layer F.Cu) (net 5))
 (segment (start 111.955 99.19) (end 111.825 99.06) (width 0.5) (layer F.Cu) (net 5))
 (segment (start 111.955 100.015) (end 111.955 99.19) (width 0.5) (layer F.Cu) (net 5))
 (segment (start 108.67 99.19) (end 107.95 99.91) (width 2) (layer F.Cu) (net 5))
 (segment (start 111.955 99.19) (end 108.67 99.19) (width 2) (layer F.Cu) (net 5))
 (segment (start 114.46 81.915) (end 116.04 81.915) (width 0.5) (layer F.Cu) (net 6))
 (segment (start 119.265 81.915) (end 117.64 81.915) (width 0.5) (layer F.Cu) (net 7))
 (segment (start 119.265 83.82) (end 117.64 83.82) (width 0.5) (layer F.Cu) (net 8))
 (segment (start 115.405 83.185) (end 114.46 83.185) (width 0.5) (layer F.Cu) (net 9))
 (segment (start 116.04 83.82) (end 115.405 83.185) (width 0.5) (layer F.Cu) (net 9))
 (segment (start 115.265 78.59) (end 115.115 78.74) (width 0.5) (layer F.Cu) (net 13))
 (segment (start 115.265 75.825) (end 115.265 78.59) (width 0.5) (layer F.Cu) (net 13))
 (segment (start 130.81 90.805) (end 132.715 92.71) (width 1.5) (layer F.Cu) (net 18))
 (segment (start 123.19 92.71) (end 122.555 93.345) (width 1.5) (layer F.Cu) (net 20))
 (segment (start 123.19 90.805) (end 123.19 92.71) (width 1.5) (layer F.Cu) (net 20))
 (segment (start 128.27 93.23) (end 128.905 93.865) (width 0.5) (layer F.Cu) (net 14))
 (segment (start 128.27 90.805) (end 128.27 93.23) (width 0.5) (layer F.Cu) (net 14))
 (segment (start 128.905 93.865) (end 130.81 93.865) (width 0.5) (layer F.Cu) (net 14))
 (segment (start 132.715 95.77) (end 130.81 93.865) (width 0.5) (layer F.Cu) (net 14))
 (segment (start 132.715 97.63) (end 132.715 95.77) (width 0.5) (layer F.Cu) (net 14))
 (segment (start 107.315 81.915) (end 109.06 81.915) (width 0.5) (layer F.Cu) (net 15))
 (segment (start 127 93.865) (end 125.095 93.865) (width 0.5) (layer F.Cu) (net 16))
 (segment (start 125.095 91.44) (end 125.73 90.805) (width 0.5) (layer F.Cu) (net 16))
 (segment (start 125.095 93.865) (end 125.095 91.44) (width 0.5) (layer F.Cu) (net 16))
 (segment (start 123.19 95.77) (end 125.095 93.865) (width 0.5) (layer F.Cu) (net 16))
 (segment (start 123.19 97.63) (end 123.19 95.77) (width 0.5) (layer F.Cu) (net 16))
 (segment (start 112.51 104.14) (end 113.55 104.14) (width 0.5) (layer F.Cu) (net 17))
 (segment (start 112.51 102.47) (end 111.955 101.915) (width 0.5) (layer F.Cu) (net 17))
 (segment (start 112.51 104.14) (end 112.51 102.47) (width 0.5) (layer F.Cu) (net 17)))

